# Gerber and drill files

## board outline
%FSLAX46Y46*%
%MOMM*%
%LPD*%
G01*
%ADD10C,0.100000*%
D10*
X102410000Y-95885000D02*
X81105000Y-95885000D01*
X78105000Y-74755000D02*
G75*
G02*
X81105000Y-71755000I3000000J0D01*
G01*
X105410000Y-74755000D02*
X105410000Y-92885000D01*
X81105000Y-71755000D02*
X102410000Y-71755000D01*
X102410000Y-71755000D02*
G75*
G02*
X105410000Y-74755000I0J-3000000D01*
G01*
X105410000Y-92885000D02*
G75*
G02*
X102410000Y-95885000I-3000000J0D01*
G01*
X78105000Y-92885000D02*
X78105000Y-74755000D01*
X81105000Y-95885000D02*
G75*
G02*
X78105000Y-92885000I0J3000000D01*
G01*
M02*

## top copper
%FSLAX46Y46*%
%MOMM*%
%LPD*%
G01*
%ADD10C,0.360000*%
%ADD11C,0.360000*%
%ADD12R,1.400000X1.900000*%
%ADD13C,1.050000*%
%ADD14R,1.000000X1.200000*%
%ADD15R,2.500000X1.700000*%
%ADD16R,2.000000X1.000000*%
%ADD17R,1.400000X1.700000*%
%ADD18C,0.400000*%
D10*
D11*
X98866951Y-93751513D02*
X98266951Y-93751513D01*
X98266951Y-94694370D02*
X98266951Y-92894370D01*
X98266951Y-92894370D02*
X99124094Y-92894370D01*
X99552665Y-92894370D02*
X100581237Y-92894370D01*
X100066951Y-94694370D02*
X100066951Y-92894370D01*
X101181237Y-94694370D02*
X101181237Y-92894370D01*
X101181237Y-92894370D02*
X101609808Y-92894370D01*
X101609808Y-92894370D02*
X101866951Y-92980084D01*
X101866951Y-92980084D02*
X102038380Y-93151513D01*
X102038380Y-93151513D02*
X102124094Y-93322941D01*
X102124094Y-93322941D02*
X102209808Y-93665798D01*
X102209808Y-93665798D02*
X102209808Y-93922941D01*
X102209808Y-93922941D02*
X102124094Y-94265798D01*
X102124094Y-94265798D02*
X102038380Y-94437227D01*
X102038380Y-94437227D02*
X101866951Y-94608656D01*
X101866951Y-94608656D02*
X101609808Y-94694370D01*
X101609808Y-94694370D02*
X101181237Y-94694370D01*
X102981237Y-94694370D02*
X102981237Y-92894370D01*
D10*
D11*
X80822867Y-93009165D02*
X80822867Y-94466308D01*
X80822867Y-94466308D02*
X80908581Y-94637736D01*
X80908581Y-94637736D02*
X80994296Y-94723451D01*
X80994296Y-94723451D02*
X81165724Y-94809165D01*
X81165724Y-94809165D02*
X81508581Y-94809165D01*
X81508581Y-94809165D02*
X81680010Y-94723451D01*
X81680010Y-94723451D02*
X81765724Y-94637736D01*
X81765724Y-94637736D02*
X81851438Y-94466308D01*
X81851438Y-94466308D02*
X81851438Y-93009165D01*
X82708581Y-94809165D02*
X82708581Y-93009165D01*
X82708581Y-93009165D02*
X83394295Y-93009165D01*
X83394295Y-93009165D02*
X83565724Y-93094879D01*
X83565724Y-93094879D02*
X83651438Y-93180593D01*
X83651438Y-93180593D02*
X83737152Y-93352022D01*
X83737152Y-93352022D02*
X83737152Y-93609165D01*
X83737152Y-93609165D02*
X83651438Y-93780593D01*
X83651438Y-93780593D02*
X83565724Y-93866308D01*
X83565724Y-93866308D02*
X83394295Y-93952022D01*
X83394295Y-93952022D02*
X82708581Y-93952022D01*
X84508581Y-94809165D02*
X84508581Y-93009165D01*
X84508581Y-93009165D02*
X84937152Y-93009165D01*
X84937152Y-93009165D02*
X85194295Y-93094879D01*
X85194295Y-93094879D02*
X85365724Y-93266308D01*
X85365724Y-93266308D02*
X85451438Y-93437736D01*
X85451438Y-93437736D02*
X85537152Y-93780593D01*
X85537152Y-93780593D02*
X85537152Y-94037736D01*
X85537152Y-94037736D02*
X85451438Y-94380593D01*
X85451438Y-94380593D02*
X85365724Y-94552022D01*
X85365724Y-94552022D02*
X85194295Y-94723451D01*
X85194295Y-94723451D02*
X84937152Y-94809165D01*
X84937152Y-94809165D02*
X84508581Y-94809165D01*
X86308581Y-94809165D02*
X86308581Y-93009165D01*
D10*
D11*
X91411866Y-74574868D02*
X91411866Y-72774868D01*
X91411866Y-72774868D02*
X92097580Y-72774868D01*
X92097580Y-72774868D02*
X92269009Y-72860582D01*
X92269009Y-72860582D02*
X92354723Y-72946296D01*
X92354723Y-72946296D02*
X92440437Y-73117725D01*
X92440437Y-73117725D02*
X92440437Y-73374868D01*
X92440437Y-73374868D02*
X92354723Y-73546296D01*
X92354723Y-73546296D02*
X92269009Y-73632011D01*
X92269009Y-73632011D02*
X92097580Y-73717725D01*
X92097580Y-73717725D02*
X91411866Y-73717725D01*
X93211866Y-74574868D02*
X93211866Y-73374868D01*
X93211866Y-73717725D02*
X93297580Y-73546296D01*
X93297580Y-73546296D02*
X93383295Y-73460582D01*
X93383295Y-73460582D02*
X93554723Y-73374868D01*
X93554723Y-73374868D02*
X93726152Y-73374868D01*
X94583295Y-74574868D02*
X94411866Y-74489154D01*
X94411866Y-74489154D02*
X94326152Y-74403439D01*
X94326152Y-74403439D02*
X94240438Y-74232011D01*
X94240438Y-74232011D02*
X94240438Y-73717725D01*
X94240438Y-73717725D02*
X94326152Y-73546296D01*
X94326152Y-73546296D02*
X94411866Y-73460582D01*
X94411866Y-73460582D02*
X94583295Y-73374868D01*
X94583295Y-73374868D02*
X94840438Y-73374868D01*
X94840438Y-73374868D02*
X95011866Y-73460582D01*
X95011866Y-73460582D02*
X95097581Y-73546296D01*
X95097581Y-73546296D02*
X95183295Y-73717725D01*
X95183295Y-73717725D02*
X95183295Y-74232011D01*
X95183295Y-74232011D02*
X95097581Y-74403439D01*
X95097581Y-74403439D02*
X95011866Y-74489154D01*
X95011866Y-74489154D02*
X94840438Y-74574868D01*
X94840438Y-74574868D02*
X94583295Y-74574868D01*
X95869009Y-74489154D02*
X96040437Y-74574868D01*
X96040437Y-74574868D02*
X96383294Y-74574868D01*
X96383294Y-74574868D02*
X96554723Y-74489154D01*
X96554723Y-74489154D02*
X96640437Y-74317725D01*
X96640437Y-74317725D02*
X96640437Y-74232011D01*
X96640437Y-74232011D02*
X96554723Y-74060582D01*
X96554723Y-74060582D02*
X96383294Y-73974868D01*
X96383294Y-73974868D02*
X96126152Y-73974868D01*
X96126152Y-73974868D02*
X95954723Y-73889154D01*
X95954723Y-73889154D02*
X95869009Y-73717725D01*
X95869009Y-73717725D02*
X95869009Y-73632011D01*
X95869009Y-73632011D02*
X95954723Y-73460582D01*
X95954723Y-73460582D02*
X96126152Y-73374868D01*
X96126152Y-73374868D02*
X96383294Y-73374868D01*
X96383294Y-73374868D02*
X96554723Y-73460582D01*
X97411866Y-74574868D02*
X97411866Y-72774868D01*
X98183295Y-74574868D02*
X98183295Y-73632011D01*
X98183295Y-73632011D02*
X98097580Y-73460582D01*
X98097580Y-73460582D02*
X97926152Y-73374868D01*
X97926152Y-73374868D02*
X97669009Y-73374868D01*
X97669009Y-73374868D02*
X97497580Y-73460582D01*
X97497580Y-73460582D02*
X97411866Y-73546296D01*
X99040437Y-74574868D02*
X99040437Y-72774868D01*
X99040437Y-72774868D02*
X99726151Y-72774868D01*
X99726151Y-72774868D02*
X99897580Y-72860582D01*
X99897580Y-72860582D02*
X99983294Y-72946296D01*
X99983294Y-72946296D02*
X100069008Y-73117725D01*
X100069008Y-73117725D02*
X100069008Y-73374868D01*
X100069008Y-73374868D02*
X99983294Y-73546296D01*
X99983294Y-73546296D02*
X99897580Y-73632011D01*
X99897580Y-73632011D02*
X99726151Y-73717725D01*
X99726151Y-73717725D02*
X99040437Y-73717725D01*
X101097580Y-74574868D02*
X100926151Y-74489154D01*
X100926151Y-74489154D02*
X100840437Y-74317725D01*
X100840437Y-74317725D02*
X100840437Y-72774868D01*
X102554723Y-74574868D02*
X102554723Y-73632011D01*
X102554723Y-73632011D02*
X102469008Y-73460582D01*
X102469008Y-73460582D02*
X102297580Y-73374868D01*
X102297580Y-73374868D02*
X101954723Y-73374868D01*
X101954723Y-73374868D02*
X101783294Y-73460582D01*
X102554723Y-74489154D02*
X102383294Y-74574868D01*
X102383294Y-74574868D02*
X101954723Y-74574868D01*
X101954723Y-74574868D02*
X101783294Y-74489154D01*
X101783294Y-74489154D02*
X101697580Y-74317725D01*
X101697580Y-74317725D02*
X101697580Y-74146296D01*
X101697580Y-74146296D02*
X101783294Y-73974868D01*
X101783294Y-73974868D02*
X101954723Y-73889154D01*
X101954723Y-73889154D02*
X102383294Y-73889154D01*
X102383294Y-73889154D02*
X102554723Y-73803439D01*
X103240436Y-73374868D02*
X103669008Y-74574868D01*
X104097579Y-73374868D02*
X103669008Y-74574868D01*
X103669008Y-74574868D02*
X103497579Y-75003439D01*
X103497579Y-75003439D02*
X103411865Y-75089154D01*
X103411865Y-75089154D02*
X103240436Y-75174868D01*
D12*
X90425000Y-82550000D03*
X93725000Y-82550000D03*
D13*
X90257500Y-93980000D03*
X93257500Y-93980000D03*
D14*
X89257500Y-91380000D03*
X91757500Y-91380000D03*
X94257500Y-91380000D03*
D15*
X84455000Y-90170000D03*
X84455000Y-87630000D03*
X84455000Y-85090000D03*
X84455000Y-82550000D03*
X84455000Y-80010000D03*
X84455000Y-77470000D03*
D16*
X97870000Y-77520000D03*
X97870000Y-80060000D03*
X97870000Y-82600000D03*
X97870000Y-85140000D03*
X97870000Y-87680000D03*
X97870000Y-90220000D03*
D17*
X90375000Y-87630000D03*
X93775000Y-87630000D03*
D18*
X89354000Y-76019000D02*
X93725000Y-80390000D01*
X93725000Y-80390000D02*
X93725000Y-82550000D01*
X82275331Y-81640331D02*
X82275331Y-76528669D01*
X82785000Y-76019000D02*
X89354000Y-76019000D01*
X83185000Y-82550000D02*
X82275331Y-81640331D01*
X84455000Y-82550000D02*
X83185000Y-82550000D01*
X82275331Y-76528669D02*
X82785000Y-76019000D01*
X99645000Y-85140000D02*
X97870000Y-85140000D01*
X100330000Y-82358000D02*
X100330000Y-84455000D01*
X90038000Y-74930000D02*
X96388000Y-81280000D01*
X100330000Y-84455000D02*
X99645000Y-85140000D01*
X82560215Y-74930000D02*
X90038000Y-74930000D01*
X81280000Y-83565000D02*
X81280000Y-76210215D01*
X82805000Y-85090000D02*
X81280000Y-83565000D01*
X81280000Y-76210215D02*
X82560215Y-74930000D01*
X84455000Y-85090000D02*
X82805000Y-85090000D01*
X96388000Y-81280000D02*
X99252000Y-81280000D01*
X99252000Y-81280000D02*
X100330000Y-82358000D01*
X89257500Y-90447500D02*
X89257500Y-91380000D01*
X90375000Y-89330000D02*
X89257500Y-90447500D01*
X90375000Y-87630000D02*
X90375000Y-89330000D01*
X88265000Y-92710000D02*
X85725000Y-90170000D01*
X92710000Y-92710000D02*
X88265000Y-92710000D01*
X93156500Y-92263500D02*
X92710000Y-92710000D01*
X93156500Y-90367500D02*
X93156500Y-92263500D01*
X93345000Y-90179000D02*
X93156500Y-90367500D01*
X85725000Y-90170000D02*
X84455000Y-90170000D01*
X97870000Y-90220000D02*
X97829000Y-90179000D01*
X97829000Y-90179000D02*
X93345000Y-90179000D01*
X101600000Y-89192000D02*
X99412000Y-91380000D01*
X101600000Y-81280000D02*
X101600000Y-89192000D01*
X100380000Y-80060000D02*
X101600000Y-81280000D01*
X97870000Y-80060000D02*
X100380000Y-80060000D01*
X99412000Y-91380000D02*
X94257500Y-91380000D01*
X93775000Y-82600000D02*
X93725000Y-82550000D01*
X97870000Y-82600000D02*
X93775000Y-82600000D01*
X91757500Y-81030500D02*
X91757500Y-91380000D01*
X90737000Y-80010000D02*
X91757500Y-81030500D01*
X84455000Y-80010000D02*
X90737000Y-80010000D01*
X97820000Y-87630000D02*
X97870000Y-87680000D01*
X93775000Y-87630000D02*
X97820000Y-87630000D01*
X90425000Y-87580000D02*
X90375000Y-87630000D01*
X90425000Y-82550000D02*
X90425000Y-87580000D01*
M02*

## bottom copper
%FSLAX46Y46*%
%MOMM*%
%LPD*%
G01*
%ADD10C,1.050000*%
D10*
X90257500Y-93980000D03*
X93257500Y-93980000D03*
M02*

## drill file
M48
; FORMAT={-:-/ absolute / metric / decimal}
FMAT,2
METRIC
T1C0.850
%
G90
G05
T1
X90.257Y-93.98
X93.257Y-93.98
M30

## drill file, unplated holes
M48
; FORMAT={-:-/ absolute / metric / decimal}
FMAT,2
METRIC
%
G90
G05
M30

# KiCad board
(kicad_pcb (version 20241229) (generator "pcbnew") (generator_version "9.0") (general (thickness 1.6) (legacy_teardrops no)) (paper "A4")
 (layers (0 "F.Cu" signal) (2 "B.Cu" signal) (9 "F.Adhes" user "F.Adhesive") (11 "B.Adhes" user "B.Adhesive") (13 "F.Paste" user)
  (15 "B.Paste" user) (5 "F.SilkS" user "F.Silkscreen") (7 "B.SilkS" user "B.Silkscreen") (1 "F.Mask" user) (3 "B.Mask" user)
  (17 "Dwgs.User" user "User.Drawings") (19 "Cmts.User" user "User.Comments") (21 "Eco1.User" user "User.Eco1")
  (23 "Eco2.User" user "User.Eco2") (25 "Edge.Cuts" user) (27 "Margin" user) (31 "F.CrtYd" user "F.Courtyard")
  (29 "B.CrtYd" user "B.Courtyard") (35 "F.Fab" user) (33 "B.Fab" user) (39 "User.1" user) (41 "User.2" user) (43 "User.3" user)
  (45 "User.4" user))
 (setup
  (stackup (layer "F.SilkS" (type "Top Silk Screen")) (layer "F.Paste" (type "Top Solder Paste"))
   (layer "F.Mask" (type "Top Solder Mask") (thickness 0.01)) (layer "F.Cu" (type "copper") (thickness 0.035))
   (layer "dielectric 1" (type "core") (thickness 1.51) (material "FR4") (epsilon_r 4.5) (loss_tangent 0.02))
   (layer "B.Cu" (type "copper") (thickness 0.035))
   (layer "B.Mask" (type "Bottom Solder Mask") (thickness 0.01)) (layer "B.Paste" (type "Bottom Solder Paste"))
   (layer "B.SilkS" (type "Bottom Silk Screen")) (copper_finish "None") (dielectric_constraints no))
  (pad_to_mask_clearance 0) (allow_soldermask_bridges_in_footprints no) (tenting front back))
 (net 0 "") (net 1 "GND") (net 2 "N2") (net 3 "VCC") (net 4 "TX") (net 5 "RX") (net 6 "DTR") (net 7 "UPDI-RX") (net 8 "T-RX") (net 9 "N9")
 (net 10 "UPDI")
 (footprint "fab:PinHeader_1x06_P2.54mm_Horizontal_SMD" (layer "F.Cu") (at 84.455 90.17 180)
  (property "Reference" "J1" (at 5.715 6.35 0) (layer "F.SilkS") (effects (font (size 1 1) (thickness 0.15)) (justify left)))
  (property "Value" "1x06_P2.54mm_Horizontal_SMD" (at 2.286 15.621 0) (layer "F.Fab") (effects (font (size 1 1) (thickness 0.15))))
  (pad "1" smd rect (at 0 0 180) (size 2.5 1.7) (layers "F.Cu" "F.Mask" "F.Paste") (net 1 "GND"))
  (pad "2" smd rect (at 0 2.54 180) (size 2.5 1.7) (layers "F.Cu" "F.Mask" "F.Paste") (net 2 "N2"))
  (pad "3" smd rect (at 0 5.08 180) (size 2.5 1.7) (layers "F.Cu" "F.Mask" "F.Paste") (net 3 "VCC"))
  (pad "4" smd rect (at 0 7.62 180) (size 2.5 1.7) (layers "F.Cu" "F.Mask" "F.Paste") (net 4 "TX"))
  (pad "5" smd rect (at 0 10.16 180) (size 2.5 1.7) (layers "F.Cu" "F.Mask" "F.Paste") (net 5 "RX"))
  (pad "6" smd rect (at 0 12.7 180) (size 2.5 1.7) (layers "F.Cu" "F.Mask" "F.Paste") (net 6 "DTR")))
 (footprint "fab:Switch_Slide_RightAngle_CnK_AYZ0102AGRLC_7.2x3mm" (layer "F.Cu") (at 91.7575 93.98)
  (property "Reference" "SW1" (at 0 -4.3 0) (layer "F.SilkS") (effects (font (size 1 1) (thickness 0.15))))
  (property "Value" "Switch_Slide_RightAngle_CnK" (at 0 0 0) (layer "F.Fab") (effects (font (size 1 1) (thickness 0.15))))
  (pad "" thru_hole circle (at -1.5 0 90) (size 1.05 1.05) (drill 0.85) (layers "*.Cu" "*.Mask") (remove_unused_layers no))
  (pad "" thru_hole circle (at 1.5 0) (size 1.05 1.05) (drill 0.85) (layers "*.Cu" "*.Mask") (remove_unused_layers no))
  (pad "1" smd rect (at -2.5 -2.6) (size 1 1.2) (layers "F.Cu" "F.Mask" "F.Paste") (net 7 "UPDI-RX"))
  (pad "2" smd rect (at 0 -2.6) (size 1 1.2) (layers "F.Cu" "F.Mask" "F.Paste") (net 5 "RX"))
  (pad "3" smd rect (at 2.5 -2.6) (size 1 1.2) (layers "F.Cu" "F.Mask" "F.Paste") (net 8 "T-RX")))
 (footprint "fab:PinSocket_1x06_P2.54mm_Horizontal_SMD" (layer "F.Cu") (at 97.87 77.52)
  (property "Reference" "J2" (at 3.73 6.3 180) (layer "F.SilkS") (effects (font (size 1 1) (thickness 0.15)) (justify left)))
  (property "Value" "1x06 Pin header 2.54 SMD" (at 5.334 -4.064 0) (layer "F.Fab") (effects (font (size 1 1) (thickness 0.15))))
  (pad "1" smd rect (at 0 0) (size 2 1) (layers "F.Cu" "F.Mask" "F.Paste") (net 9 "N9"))
  (pad "2" smd rect (at 0 2.54) (size 2 1) (layers "F.Cu" "F.Mask" "F.Paste") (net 8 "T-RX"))
  (pad "3" smd rect (at 0 5.08) (size 2 1) (layers "F.Cu" "F.Mask" "F.Paste") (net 4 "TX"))
  (pad "4" smd rect (at 0 7.62) (size 2 1) (layers "F.Cu" "F.Mask" "F.Paste") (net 3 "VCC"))
  (pad "5" smd rect (at 0 10.16) (size 2 1) (layers "F.Cu" "F.Mask" "F.Paste") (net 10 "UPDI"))
  (pad "6" smd rect (at 0 12.7) (size 2 1) (layers "F.Cu" "F.Mask" "F.Paste") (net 1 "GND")))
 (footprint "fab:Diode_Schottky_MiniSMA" (layer "F.Cu") (at 92.075 82.55 180)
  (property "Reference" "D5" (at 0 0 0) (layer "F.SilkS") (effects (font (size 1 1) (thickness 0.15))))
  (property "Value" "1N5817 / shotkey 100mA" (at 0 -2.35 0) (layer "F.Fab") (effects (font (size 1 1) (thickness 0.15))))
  (pad "1" smd rect (at -1.65 0 180) (size 1.4 1.9) (layers "F.Cu" "F.Mask" "F.Paste") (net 4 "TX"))
  (pad "2" smd rect (at 1.65 0 180) (size 1.4 1.9) (layers "F.Cu" "F.Mask" "F.Paste") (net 7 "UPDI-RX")))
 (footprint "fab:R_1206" (layer "F.Cu") (at 92.075 87.63)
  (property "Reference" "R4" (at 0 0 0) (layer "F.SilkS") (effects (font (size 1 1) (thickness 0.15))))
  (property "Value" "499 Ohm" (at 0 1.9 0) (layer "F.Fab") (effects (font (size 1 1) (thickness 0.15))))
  (pad "1" smd rect (at -1.7 0) (size 1.4 1.7) (layers "F.Cu" "F.Mask" "F.Paste") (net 7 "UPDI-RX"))
  (pad "2" smd rect (at 1.7 0) (size 1.4 1.7) (layers "F.Cu" "F.Mask" "F.Paste") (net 10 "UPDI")))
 (gr_line (start 102.41 95.885) (end 81.105 95.885) (stroke (width 0.1) (type default)) (layer "Edge.Cuts"))
 (gr_arc (start 78.105 74.755) (mid 78.98368 72.63368) (end 81.105 71.755) (stroke (width 0.1) (type default)) (layer "Edge.Cuts"))
 (gr_line (start 105.41 74.755) (end 105.41 92.885) (stroke (width 0.1) (type default)) (layer "Edge.Cuts"))
 (gr_line (start 81.105 71.755) (end 102.41 71.755) (stroke (width 0.1) (type default)) (layer "Edge.Cuts"))
 (gr_arc (start 102.41 71.755) (mid 104.53132 72.63368) (end 105.41 74.755) (stroke (width 0.1) (type default)) (layer "Edge.Cuts"))
 (gr_arc (start 105.41 92.885) (mid 104.53132 95.00632) (end 102.41 95.885) (stroke (width 0.1) (type default)) (layer "Edge.Cuts"))
 (gr_line (start 78.105 92.885) (end 78.105 74.755) (stroke (width 0.1) (type default)) (layer "Edge.Cuts"))
 (gr_arc (start 81.105 95.885) (mid 78.98368 95.00632) (end 78.105 92.885) (stroke (width 0.1) (type default)) (layer "Edge.Cuts"))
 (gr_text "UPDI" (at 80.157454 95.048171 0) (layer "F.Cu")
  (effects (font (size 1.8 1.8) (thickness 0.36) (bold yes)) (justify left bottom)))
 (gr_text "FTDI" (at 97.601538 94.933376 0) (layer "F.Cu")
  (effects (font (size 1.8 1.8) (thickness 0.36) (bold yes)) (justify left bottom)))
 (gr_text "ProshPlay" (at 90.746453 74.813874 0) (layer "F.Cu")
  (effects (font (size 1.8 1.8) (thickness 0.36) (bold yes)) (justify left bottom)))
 (segment (start 93.725 80.39) (end 93.725 82.55) (width 0.4) (layer "F.Cu") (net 4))
 (segment (start 82.785 76.019) (end 89.354 76.019) (width 0.4) (layer "F.Cu") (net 4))
 (segment (start 82.275331 81.640331) (end 82.275331 76.528669) (width 0.4) (layer "F.Cu") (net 4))
 (segment (start 82.275331 76.528669) (end 82.785 76.019) (width 0.4) (layer "F.Cu") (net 4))
 (segment (start 97.87 82.6) (end 93.775 82.6) (width 0.4) (layer "F.Cu") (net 4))
 (segment (start 89.354 76.019) (end 93.725 80.39) (width 0.4) (layer "F.Cu") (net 4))
 (segment (start 93.775 82.6) (end 93.725 82.55) (width 0.4) (layer "F.Cu") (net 4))
 (segment (start 84.455 82.55) (end 83.185 82.55) (width 0.4) (layer "F.Cu") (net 4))
 (segment (start 83.185 82.55) (end 82.275331 81.640331) (width 0.4) (layer "F.Cu") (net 4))
 (segment (start 93.1565 92.2635) (end 92.71 92.71) (width 0.4) (layer "F.Cu") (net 1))
 (segment (start 93.1565 90.3675) (end 93.1565 92.2635) (width 0.4) (layer "F.Cu") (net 1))
 (segment (start 88.265 92.71) (end 85.725 90.17) (width 0.4) (layer "F.Cu") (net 1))
 (segment (start 97.87 90.22) (end 97.829 90.179) (width 0.4) (layer "F.Cu") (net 1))
 (segment (start 92.71 92.71) (end 88.265 92.71) (width 0.4) (layer "F.Cu") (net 1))
 (segment (start 85.725 90.17) (end 84.455 90.17) (width 0.4) (layer "F.Cu") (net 1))
 (segment (start 93.345 90.179) (end 93.1565 90.3675) (width 0.4) (layer "F.Cu") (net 1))
 (segment (start 97.829 90.179) (end 93.345 90.179) (width 0.4) (layer "F.Cu") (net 1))
 (segment (start 82.805 85.09) (end 81.28 83.565) (width 0.4) (layer "F.Cu") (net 3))
 (segment (start 84.455 85.09) (end 82.805 85.09) (width 0.4) (layer "F.Cu") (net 3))
 (segment (start 81.28 83.565) (end 81.28 76.210215) (width 0.4) (layer "F.Cu") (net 3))
 (segment (start 99.252 81.28) (end 100.33 82.358) (width 0.4) (layer "F.Cu") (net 3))
 (segment (start 82.560215 74.93) (end 90.038 74.93) (width 0.4) (layer "F.Cu") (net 3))
 (segment (start 81.28 76.210215) (end 82.560215 74.93) (width 0.4) (layer "F.Cu") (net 3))
 (segment (start 100.33 84.455) (end 99.645 85.14) (width 0.4) (layer "F.Cu") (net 3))
 (segment (start 99.645 85.14) (end 97.87 85.14) (width 0.4) (layer "F.Cu") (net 3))
 (segment (start 96.388 81.28) (end 99.252 81.28) (width 0.4) (layer "F.Cu") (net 3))
 (segment (start 90.038 74.93) (end 96.388 81.28) (width 0.4) (layer "F.Cu") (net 3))
 (segment (start 100.33 82.358) (end 100.33 84.455) (width 0.4) (layer "F.Cu") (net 3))
 (segment (start 84.455 80.01) (end 90.737 80.01) (width 0.4) (layer "F.Cu") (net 5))
 (segment (start 91.7575 81.0305) (end 91.7575 91.38) (width 0.4) (layer "F.Cu") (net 5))
 (segment (start 90.737 80.01) (end 91.7575 81.0305) (width 0.4) (layer "F.Cu") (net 5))
 (segment (start 93.775 87.63) (end 97.82 87.63) (width 0.4) (layer "F.Cu") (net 10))
 (segment (start 97.82 87.63) (end 97.87 87.68) (width 0.4) (layer "F.Cu") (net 10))
 (segment (start 101.6 89.192) (end 99.412 91.38) (width 0.4) (layer "F.Cu") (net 8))
 (segment (start 101.6 81.28) (end 101.6 89.192) (width 0.4) (layer "F.Cu") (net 8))
 (segment (start 99.412 91.38) (end 94.2575 91.38) (width 0.4) (layer "F.Cu") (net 8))
 (segment (start 97.87 80.06) (end 100.38 80.06) (width 0.4) (layer "F.Cu") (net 8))
 (segment (start 100.38 80.06) (end 101.6 81.28) (width 0.4) (layer "F.Cu") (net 8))
 (segment (start 90.425 87.58) (end 90.375 87.63) (width 0.4) (layer "F.Cu") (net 7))
 (segment (start 90.375 87.63) (end 90.375 89.33) (width 0.4) (layer "F.Cu") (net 7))
 (segment (start 90.375 89.33) (end 89.2575 90.4475) (width 0.4) (layer "F.Cu") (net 7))
 (segment (start 90.425 82.55) (end 90.425 87.58) (width 0.4) (layer "F.Cu") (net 7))
 (segment (start 89.2575 90.4475) (end 89.2575 91.38) (width 0.4) (layer "F.Cu") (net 7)))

